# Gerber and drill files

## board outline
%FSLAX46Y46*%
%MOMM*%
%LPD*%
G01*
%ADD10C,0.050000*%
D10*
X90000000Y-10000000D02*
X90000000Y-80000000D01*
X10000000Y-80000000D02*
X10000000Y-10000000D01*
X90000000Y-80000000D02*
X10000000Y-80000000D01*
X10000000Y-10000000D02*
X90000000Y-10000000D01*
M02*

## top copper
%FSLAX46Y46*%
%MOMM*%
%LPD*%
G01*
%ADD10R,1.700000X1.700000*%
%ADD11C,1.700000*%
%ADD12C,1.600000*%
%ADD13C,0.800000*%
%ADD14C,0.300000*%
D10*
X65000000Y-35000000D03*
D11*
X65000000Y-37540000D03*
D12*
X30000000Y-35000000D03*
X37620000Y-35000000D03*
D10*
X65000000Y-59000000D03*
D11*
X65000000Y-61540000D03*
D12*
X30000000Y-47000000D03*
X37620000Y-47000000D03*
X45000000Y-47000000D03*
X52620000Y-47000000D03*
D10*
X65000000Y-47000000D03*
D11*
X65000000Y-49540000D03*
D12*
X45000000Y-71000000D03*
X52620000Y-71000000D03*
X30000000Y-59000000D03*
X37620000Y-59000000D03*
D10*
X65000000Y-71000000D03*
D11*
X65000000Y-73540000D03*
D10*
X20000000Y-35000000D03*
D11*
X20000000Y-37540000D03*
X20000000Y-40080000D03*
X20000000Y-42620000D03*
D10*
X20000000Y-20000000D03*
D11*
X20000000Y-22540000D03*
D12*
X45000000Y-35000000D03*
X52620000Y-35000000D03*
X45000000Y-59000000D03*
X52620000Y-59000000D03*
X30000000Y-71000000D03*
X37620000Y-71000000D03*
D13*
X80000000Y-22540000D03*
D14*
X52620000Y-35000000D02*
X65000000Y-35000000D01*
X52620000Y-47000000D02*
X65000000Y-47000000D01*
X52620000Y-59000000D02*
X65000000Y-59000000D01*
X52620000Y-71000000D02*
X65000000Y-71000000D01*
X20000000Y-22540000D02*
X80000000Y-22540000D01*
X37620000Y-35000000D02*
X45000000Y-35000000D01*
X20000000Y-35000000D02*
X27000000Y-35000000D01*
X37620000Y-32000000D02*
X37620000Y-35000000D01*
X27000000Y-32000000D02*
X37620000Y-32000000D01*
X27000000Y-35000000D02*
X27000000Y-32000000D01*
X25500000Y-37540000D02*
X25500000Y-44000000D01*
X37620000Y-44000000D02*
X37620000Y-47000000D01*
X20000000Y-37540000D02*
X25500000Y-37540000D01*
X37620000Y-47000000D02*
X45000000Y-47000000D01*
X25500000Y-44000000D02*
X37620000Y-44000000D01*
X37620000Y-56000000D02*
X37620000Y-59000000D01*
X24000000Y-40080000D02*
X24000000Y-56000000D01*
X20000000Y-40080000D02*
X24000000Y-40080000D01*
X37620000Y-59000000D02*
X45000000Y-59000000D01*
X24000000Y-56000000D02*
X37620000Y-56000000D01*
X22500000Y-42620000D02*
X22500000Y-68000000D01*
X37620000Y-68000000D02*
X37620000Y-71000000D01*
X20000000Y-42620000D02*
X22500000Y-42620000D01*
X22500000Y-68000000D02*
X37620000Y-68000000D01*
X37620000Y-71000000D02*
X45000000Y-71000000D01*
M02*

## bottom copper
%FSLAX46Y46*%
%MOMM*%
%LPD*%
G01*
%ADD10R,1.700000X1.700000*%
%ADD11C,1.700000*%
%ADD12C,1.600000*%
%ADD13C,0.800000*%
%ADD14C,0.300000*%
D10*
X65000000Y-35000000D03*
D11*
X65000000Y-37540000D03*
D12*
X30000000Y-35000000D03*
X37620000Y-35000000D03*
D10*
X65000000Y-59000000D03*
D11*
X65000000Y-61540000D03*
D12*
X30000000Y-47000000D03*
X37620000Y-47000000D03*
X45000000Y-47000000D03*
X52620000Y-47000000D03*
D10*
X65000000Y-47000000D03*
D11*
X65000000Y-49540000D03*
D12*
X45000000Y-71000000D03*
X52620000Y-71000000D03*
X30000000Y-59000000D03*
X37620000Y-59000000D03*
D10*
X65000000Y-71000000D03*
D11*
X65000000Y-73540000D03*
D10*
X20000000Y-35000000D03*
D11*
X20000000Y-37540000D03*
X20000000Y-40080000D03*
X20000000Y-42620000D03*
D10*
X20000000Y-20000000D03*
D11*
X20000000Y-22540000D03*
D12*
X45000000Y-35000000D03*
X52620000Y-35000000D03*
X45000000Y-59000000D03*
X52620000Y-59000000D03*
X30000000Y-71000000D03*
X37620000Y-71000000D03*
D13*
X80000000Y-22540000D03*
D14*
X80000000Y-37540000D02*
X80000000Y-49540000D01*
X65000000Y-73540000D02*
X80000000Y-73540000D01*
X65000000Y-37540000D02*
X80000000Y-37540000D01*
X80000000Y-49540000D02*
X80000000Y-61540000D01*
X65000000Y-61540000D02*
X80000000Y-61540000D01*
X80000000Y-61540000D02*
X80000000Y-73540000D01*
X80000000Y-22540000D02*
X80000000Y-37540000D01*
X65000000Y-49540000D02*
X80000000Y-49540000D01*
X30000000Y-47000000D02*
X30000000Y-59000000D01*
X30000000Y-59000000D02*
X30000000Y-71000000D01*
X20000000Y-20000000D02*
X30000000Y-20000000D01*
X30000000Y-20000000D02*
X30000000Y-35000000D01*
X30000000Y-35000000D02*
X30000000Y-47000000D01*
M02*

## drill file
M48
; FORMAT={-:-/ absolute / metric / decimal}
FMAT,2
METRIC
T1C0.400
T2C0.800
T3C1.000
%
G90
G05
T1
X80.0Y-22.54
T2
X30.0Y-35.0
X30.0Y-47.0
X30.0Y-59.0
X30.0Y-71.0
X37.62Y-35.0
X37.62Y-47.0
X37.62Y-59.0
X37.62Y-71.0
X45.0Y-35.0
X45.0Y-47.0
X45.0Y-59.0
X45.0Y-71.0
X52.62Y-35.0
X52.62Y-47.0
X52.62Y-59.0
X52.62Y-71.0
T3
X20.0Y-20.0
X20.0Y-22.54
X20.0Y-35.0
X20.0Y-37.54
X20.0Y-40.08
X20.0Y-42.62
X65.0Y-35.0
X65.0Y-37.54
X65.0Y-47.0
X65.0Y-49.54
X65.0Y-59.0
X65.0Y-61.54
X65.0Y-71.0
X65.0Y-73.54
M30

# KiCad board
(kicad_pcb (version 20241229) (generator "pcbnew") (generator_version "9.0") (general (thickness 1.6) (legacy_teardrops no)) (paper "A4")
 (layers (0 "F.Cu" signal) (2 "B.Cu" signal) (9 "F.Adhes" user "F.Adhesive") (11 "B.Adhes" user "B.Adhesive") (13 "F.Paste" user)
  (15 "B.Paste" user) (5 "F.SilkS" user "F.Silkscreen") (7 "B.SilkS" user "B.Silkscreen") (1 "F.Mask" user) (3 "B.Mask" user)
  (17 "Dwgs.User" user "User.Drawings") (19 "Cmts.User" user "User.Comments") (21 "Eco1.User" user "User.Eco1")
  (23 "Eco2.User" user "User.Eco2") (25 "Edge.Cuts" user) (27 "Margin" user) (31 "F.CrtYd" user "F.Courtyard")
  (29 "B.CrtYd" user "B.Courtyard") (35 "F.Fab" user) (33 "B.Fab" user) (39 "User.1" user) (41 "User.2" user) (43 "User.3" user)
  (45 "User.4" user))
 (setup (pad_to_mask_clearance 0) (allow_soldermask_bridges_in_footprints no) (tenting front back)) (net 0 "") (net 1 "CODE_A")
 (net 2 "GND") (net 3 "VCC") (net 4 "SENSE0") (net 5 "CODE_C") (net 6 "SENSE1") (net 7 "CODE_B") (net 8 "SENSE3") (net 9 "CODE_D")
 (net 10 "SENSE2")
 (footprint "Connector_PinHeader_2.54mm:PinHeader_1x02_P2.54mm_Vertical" (layer "F.Cu") (at 65 35)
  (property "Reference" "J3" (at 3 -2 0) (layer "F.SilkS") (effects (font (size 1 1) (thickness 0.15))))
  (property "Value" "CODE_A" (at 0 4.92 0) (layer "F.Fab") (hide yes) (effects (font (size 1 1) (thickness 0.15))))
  (pad "1" thru_hole rect (at 0 0) (size 1.7 1.7) (drill 1) (layers "*.Cu" "*.Mask") (remove_unused_layers no) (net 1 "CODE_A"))
  (pad "2" thru_hole circle (at 0 2.54) (size 1.7 1.7) (drill 1) (layers "*.Cu" "*.Mask") (remove_unused_layers no) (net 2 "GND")))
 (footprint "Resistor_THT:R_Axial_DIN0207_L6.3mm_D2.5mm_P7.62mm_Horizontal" (layer "F.Cu") (at 30 35)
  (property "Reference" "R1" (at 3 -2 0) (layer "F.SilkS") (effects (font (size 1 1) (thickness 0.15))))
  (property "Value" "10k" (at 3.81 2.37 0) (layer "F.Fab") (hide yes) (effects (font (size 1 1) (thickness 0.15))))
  (pad "1" thru_hole circle (at 0 0) (size 1.6 1.6) (drill 0.8) (layers "*.Cu" "*.Mask") (remove_unused_layers no) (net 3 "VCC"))
  (pad "2" thru_hole circle (at 7.62 0) (size 1.6 1.6) (drill 0.8) (layers "*.Cu" "*.Mask") (remove_unused_layers no) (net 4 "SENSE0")))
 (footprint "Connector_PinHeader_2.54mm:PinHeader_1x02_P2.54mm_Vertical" (layer "F.Cu") (at 65 59)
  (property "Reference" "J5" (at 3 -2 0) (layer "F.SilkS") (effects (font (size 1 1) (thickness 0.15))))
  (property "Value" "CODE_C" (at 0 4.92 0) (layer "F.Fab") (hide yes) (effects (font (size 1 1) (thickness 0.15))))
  (pad "1" thru_hole rect (at 0 0) (size 1.7 1.7) (drill 1) (layers "*.Cu" "*.Mask") (remove_unused_layers no) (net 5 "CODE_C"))
  (pad "2" thru_hole circle (at 0 2.54) (size 1.7 1.7) (drill 1) (layers "*.Cu" "*.Mask") (remove_unused_layers no) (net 2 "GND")))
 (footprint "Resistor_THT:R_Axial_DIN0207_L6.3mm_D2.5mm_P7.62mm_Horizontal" (layer "F.Cu") (at 30 47)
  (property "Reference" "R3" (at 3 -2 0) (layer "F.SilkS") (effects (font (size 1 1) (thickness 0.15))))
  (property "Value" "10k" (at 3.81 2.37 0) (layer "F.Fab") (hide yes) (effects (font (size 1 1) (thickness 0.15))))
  (pad "1" thru_hole circle (at 0 0) (size 1.6 1.6) (drill 0.8) (layers "*.Cu" "*.Mask") (remove_unused_layers no) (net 3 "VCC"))
  (pad "2" thru_hole circle (at 7.62 0) (size 1.6 1.6) (drill 0.8) (layers "*.Cu" "*.Mask") (remove_unused_layers no) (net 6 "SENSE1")))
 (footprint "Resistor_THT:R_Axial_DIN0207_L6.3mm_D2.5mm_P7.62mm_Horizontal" (layer "F.Cu") (at 45 47)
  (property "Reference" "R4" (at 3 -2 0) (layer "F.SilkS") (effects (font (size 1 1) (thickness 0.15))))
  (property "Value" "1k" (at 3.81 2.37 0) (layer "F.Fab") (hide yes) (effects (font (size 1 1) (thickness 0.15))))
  (pad "1" thru_hole circle (at 0 0) (size 1.6 1.6) (drill 0.8) (layers "*.Cu" "*.Mask") (remove_unused_layers no) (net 6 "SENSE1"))
  (pad "2" thru_hole circle (at 7.62 0) (size 1.6 1.6) (drill 0.8) (layers "*.Cu" "*.Mask") (remove_unused_layers no) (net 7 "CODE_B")))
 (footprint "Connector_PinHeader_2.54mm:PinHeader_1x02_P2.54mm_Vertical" (layer "F.Cu") (at 65 47)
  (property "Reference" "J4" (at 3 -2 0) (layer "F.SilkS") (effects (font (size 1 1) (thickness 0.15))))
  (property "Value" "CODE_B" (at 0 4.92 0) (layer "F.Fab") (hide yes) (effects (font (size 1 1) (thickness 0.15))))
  (pad "1" thru_hole rect (at 0 0) (size 1.7 1.7) (drill 1) (layers "*.Cu" "*.Mask") (remove_unused_layers no) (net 7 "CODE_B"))
  (pad "2" thru_hole circle (at 0 2.54) (size 1.7 1.7) (drill 1) (layers "*.Cu" "*.Mask") (remove_unused_layers no) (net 2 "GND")))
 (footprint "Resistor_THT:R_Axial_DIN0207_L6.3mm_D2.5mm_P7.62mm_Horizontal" (layer "F.Cu") (at 45 71)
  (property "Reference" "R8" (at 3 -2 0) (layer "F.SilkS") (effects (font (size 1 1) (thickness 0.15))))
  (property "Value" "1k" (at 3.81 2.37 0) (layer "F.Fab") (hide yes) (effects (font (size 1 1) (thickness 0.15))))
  (pad "1" thru_hole circle (at 0 0) (size 1.6 1.6) (drill 0.8) (layers "*.Cu" "*.Mask") (remove_unused_layers no) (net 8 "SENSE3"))
  (pad "2" thru_hole circle (at 7.62 0) (size 1.6 1.6) (drill 0.8) (layers "*.Cu" "*.Mask") (remove_unused_layers no) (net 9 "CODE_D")))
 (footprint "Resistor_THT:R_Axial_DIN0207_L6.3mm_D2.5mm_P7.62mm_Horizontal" (layer "F.Cu") (at 30 59)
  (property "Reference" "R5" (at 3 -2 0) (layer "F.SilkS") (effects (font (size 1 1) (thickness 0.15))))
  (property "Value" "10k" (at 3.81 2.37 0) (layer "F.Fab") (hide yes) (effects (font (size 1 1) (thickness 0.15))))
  (pad "1" thru_hole circle (at 0 0) (size 1.6 1.6) (drill 0.8) (layers "*.Cu" "*.Mask") (remove_unused_layers no) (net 3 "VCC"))
  (pad "2" thru_hole circle (at 7.62 0) (size 1.6 1.6) (drill 0.8) (layers "*.Cu" "*.Mask") (remove_unused_layers no) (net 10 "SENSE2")))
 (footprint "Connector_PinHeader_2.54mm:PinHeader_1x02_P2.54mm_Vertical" (layer "F.Cu") (at 65 71)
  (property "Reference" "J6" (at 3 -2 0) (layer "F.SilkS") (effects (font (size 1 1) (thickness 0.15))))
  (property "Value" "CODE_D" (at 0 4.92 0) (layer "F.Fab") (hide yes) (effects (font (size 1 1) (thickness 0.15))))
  (pad "1" thru_hole rect (at 0 0) (size 1.7 1.7) (drill 1) (layers "*.Cu" "*.Mask") (remove_unused_layers no) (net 9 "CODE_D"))
  (pad "2" thru_hole circle (at 0 2.54) (size 1.7 1.7) (drill 1) (layers "*.Cu" "*.Mask") (remove_unused_layers no) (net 2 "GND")))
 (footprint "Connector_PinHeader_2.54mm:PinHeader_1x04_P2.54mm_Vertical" (layer "F.Cu") (at 20 35)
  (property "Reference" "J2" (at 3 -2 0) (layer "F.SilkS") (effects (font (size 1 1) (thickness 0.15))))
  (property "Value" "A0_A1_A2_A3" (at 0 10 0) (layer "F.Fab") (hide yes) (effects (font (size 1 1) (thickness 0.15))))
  (pad "1" thru_hole rect (at 0 0) (size 1.7 1.7) (drill 1) (layers "*.Cu" "*.Mask") (remove_unused_layers no) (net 4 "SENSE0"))
  (pad "2" thru_hole circle (at 0 2.54) (size 1.7 1.7) (drill 1) (layers "*.Cu" "*.Mask") (remove_unused_layers no) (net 6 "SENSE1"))
  (pad "3" thru_hole circle (at 0 5.08) (size 1.7 1.7) (drill 1) (layers "*.Cu" "*.Mask") (remove_unused_layers no) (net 10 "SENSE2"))
  (pad "4" thru_hole circle (at 0 7.62) (size 1.7 1.7) (drill 1) (layers "*.Cu" "*.Mask") (remove_unused_layers no) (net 8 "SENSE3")))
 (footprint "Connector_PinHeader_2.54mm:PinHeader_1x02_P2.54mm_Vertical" (layer "F.Cu") (at 20 20)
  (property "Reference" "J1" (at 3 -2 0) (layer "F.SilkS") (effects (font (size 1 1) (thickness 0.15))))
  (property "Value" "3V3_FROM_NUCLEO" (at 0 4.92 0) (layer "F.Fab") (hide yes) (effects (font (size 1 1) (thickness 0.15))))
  (pad "1" thru_hole rect (at 0 0) (size 1.7 1.7) (drill 1) (layers "*.Cu" "*.Mask") (remove_unused_layers no) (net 3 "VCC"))
  (pad "2" thru_hole circle (at 0 2.54) (size 1.7 1.7) (drill 1) (layers "*.Cu" "*.Mask") (remove_unused_layers no) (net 2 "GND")))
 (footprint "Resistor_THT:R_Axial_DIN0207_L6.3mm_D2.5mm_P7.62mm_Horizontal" (layer "F.Cu") (at 45 35)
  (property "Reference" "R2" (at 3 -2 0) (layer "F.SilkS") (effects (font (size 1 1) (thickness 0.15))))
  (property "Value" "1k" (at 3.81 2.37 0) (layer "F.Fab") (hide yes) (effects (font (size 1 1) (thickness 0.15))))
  (pad "1" thru_hole circle (at 0 0) (size 1.6 1.6) (drill 0.8) (layers "*.Cu" "*.Mask") (remove_unused_layers no) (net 4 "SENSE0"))
  (pad "2" thru_hole circle (at 7.62 0) (size 1.6 1.6) (drill 0.8) (layers "*.Cu" "*.Mask") (remove_unused_layers no) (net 1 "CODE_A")))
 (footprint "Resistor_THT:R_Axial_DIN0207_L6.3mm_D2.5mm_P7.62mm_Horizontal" (layer "F.Cu") (at 45 59)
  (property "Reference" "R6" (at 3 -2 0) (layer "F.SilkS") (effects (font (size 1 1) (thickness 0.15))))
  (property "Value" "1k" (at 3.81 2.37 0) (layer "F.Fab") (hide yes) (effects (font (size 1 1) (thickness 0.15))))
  (pad "1" thru_hole circle (at 0 0) (size 1.6 1.6) (drill 0.8) (layers "*.Cu" "*.Mask") (remove_unused_layers no) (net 10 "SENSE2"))
  (pad "2" thru_hole circle (at 7.62 0) (size 1.6 1.6) (drill 0.8) (layers "*.Cu" "*.Mask") (remove_unused_layers no) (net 5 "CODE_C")))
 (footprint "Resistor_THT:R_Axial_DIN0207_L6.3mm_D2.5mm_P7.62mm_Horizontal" (layer "F.Cu") (at 30 71)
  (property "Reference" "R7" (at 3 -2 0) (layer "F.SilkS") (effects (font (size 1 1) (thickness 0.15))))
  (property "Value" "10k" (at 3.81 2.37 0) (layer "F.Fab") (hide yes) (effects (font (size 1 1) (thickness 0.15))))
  (pad "1" thru_hole circle (at 0 0) (size 1.6 1.6) (drill 0.8) (layers "*.Cu" "*.Mask") (remove_unused_layers no) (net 3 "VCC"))
  (pad "2" thru_hole circle (at 7.62 0) (size 1.6 1.6) (drill 0.8) (layers "*.Cu" "*.Mask") (remove_unused_layers no) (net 8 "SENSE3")))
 (gr_line (start 90 10) (end 90 80) (stroke (width 0.05) (type default)) (layer "Edge.Cuts"))
 (gr_line (start 10 80) (end 10 10) (stroke (width 0.05) (type default)) (layer "Edge.Cuts"))
 (gr_line (start 90 80) (end 10 80) (stroke (width 0.05) (type default)) (layer "Edge.Cuts"))
 (gr_line (start 10 10) (end 90 10) (stroke (width 0.05) (type default)) (layer "Edge.Cuts"))
 (segment (start 52.62 35) (end 65 35) (width 0.3) (layer "F.Cu") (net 1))
 (segment (start 52.62 47) (end 65 47) (width 0.3) (layer "F.Cu") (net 7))
 (segment (start 52.62 59) (end 65 59) (width 0.3) (layer "F.Cu") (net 5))
 (segment (start 52.62 71) (end 65 71) (width 0.3) (layer "F.Cu") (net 9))
 (segment (start 20 22.54) (end 80 22.54) (width 0.3) (layer "F.Cu") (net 2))
 (via (at 80 22.54) (size 0.8) (drill 0.4) (layers "F.Cu" "B.Cu") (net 2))
 (segment (start 80 37.54) (end 80 49.54) (width 0.3) (layer "B.Cu") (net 2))
 (segment (start 65 73.54) (end 80 73.54) (width 0.3) (layer "B.Cu") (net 2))
 (segment (start 65 37.54) (end 80 37.54) (width 0.3) (layer "B.Cu") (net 2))
 (segment (start 80 49.54) (end 80 61.54) (width 0.3) (layer "B.Cu") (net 2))
 (segment (start 65 61.54) (end 80 61.54) (width 0.3) (layer "B.Cu") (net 2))
 (segment (start 80 61.54) (end 80 73.54) (width 0.3) (layer "B.Cu") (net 2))
 (segment (start 80 22.54) (end 80 37.54) (width 0.3) (layer "B.Cu") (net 2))
 (segment (start 65 49.54) (end 80 49.54) (width 0.3) (layer "B.Cu") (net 2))
 (segment (start 37.62 35) (end 45 35) (width 0.3) (layer "F.Cu") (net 4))
 (segment (start 20 35) (end 27 35) (width 0.3) (layer "F.Cu") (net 4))
 (segment (start 37.62 32) (end 37.62 35) (width 0.3) (layer "F.Cu") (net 4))
 (segment (start 27 32) (end 37.62 32) (width 0.3) (layer "F.Cu") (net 4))
 (segment (start 27 35) (end 27 32) (width 0.3) (layer "F.Cu") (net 4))
 (segment (start 25.5 37.54) (end 25.5 44) (width 0.3) (layer "F.Cu") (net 6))
 (segment (start 37.62 44) (end 37.62 47) (width 0.3) (layer "F.Cu") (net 6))
 (segment (start 20 37.54) (end 25.5 37.54) (width 0.3) (layer "F.Cu") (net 6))
 (segment (start 37.62 47) (end 45 47) (width 0.3) (layer "F.Cu") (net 6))
 (segment (start 25.5 44) (end 37.62 44) (width 0.3) (layer "F.Cu") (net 6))
 (segment (start 37.62 56) (end 37.62 59) (width 0.3) (layer "F.Cu") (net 10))
 (segment (start 24 40.08) (end 24 56) (width 0.3) (layer "F.Cu") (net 10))
 (segment (start 20 40.08) (end 24 40.08) (width 0.3) (layer "F.Cu") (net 10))
 (segment (start 37.62 59) (end 45 59) (width 0.3) (layer "F.Cu") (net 10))
 (segment (start 24 56) (end 37.62 56) (width 0.3) (layer "F.Cu") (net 10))
 (segment (start 22.5 42.62) (end 22.5 68) (width 0.3) (layer "F.Cu") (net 8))
 (segment (start 37.62 68) (end 37.62 71) (width 0.3) (layer "F.Cu") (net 8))
 (segment (start 20 42.62) (end 22.5 42.62) (width 0.3) (layer "F.Cu") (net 8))
 (segment (start 22.5 68) (end 37.62 68) (width 0.3) (layer "F.Cu") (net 8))
 (segment (start 37.62 71) (end 45 71) (width 0.3) (layer "F.Cu") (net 8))
 (segment (start 30 47) (end 30 59) (width 0.3) (layer "B.Cu") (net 3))
 (segment (start 30 59) (end 30 71) (width 0.3) (layer "B.Cu") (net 3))
 (segment (start 20 20) (end 30 20) (width 0.3) (layer "B.Cu") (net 3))
 (segment (start 30 20) (end 30 35) (width 0.3) (layer "B.Cu") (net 3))
 (segment (start 30 35) (end 30 47) (width 0.3) (layer "B.Cu") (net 3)))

